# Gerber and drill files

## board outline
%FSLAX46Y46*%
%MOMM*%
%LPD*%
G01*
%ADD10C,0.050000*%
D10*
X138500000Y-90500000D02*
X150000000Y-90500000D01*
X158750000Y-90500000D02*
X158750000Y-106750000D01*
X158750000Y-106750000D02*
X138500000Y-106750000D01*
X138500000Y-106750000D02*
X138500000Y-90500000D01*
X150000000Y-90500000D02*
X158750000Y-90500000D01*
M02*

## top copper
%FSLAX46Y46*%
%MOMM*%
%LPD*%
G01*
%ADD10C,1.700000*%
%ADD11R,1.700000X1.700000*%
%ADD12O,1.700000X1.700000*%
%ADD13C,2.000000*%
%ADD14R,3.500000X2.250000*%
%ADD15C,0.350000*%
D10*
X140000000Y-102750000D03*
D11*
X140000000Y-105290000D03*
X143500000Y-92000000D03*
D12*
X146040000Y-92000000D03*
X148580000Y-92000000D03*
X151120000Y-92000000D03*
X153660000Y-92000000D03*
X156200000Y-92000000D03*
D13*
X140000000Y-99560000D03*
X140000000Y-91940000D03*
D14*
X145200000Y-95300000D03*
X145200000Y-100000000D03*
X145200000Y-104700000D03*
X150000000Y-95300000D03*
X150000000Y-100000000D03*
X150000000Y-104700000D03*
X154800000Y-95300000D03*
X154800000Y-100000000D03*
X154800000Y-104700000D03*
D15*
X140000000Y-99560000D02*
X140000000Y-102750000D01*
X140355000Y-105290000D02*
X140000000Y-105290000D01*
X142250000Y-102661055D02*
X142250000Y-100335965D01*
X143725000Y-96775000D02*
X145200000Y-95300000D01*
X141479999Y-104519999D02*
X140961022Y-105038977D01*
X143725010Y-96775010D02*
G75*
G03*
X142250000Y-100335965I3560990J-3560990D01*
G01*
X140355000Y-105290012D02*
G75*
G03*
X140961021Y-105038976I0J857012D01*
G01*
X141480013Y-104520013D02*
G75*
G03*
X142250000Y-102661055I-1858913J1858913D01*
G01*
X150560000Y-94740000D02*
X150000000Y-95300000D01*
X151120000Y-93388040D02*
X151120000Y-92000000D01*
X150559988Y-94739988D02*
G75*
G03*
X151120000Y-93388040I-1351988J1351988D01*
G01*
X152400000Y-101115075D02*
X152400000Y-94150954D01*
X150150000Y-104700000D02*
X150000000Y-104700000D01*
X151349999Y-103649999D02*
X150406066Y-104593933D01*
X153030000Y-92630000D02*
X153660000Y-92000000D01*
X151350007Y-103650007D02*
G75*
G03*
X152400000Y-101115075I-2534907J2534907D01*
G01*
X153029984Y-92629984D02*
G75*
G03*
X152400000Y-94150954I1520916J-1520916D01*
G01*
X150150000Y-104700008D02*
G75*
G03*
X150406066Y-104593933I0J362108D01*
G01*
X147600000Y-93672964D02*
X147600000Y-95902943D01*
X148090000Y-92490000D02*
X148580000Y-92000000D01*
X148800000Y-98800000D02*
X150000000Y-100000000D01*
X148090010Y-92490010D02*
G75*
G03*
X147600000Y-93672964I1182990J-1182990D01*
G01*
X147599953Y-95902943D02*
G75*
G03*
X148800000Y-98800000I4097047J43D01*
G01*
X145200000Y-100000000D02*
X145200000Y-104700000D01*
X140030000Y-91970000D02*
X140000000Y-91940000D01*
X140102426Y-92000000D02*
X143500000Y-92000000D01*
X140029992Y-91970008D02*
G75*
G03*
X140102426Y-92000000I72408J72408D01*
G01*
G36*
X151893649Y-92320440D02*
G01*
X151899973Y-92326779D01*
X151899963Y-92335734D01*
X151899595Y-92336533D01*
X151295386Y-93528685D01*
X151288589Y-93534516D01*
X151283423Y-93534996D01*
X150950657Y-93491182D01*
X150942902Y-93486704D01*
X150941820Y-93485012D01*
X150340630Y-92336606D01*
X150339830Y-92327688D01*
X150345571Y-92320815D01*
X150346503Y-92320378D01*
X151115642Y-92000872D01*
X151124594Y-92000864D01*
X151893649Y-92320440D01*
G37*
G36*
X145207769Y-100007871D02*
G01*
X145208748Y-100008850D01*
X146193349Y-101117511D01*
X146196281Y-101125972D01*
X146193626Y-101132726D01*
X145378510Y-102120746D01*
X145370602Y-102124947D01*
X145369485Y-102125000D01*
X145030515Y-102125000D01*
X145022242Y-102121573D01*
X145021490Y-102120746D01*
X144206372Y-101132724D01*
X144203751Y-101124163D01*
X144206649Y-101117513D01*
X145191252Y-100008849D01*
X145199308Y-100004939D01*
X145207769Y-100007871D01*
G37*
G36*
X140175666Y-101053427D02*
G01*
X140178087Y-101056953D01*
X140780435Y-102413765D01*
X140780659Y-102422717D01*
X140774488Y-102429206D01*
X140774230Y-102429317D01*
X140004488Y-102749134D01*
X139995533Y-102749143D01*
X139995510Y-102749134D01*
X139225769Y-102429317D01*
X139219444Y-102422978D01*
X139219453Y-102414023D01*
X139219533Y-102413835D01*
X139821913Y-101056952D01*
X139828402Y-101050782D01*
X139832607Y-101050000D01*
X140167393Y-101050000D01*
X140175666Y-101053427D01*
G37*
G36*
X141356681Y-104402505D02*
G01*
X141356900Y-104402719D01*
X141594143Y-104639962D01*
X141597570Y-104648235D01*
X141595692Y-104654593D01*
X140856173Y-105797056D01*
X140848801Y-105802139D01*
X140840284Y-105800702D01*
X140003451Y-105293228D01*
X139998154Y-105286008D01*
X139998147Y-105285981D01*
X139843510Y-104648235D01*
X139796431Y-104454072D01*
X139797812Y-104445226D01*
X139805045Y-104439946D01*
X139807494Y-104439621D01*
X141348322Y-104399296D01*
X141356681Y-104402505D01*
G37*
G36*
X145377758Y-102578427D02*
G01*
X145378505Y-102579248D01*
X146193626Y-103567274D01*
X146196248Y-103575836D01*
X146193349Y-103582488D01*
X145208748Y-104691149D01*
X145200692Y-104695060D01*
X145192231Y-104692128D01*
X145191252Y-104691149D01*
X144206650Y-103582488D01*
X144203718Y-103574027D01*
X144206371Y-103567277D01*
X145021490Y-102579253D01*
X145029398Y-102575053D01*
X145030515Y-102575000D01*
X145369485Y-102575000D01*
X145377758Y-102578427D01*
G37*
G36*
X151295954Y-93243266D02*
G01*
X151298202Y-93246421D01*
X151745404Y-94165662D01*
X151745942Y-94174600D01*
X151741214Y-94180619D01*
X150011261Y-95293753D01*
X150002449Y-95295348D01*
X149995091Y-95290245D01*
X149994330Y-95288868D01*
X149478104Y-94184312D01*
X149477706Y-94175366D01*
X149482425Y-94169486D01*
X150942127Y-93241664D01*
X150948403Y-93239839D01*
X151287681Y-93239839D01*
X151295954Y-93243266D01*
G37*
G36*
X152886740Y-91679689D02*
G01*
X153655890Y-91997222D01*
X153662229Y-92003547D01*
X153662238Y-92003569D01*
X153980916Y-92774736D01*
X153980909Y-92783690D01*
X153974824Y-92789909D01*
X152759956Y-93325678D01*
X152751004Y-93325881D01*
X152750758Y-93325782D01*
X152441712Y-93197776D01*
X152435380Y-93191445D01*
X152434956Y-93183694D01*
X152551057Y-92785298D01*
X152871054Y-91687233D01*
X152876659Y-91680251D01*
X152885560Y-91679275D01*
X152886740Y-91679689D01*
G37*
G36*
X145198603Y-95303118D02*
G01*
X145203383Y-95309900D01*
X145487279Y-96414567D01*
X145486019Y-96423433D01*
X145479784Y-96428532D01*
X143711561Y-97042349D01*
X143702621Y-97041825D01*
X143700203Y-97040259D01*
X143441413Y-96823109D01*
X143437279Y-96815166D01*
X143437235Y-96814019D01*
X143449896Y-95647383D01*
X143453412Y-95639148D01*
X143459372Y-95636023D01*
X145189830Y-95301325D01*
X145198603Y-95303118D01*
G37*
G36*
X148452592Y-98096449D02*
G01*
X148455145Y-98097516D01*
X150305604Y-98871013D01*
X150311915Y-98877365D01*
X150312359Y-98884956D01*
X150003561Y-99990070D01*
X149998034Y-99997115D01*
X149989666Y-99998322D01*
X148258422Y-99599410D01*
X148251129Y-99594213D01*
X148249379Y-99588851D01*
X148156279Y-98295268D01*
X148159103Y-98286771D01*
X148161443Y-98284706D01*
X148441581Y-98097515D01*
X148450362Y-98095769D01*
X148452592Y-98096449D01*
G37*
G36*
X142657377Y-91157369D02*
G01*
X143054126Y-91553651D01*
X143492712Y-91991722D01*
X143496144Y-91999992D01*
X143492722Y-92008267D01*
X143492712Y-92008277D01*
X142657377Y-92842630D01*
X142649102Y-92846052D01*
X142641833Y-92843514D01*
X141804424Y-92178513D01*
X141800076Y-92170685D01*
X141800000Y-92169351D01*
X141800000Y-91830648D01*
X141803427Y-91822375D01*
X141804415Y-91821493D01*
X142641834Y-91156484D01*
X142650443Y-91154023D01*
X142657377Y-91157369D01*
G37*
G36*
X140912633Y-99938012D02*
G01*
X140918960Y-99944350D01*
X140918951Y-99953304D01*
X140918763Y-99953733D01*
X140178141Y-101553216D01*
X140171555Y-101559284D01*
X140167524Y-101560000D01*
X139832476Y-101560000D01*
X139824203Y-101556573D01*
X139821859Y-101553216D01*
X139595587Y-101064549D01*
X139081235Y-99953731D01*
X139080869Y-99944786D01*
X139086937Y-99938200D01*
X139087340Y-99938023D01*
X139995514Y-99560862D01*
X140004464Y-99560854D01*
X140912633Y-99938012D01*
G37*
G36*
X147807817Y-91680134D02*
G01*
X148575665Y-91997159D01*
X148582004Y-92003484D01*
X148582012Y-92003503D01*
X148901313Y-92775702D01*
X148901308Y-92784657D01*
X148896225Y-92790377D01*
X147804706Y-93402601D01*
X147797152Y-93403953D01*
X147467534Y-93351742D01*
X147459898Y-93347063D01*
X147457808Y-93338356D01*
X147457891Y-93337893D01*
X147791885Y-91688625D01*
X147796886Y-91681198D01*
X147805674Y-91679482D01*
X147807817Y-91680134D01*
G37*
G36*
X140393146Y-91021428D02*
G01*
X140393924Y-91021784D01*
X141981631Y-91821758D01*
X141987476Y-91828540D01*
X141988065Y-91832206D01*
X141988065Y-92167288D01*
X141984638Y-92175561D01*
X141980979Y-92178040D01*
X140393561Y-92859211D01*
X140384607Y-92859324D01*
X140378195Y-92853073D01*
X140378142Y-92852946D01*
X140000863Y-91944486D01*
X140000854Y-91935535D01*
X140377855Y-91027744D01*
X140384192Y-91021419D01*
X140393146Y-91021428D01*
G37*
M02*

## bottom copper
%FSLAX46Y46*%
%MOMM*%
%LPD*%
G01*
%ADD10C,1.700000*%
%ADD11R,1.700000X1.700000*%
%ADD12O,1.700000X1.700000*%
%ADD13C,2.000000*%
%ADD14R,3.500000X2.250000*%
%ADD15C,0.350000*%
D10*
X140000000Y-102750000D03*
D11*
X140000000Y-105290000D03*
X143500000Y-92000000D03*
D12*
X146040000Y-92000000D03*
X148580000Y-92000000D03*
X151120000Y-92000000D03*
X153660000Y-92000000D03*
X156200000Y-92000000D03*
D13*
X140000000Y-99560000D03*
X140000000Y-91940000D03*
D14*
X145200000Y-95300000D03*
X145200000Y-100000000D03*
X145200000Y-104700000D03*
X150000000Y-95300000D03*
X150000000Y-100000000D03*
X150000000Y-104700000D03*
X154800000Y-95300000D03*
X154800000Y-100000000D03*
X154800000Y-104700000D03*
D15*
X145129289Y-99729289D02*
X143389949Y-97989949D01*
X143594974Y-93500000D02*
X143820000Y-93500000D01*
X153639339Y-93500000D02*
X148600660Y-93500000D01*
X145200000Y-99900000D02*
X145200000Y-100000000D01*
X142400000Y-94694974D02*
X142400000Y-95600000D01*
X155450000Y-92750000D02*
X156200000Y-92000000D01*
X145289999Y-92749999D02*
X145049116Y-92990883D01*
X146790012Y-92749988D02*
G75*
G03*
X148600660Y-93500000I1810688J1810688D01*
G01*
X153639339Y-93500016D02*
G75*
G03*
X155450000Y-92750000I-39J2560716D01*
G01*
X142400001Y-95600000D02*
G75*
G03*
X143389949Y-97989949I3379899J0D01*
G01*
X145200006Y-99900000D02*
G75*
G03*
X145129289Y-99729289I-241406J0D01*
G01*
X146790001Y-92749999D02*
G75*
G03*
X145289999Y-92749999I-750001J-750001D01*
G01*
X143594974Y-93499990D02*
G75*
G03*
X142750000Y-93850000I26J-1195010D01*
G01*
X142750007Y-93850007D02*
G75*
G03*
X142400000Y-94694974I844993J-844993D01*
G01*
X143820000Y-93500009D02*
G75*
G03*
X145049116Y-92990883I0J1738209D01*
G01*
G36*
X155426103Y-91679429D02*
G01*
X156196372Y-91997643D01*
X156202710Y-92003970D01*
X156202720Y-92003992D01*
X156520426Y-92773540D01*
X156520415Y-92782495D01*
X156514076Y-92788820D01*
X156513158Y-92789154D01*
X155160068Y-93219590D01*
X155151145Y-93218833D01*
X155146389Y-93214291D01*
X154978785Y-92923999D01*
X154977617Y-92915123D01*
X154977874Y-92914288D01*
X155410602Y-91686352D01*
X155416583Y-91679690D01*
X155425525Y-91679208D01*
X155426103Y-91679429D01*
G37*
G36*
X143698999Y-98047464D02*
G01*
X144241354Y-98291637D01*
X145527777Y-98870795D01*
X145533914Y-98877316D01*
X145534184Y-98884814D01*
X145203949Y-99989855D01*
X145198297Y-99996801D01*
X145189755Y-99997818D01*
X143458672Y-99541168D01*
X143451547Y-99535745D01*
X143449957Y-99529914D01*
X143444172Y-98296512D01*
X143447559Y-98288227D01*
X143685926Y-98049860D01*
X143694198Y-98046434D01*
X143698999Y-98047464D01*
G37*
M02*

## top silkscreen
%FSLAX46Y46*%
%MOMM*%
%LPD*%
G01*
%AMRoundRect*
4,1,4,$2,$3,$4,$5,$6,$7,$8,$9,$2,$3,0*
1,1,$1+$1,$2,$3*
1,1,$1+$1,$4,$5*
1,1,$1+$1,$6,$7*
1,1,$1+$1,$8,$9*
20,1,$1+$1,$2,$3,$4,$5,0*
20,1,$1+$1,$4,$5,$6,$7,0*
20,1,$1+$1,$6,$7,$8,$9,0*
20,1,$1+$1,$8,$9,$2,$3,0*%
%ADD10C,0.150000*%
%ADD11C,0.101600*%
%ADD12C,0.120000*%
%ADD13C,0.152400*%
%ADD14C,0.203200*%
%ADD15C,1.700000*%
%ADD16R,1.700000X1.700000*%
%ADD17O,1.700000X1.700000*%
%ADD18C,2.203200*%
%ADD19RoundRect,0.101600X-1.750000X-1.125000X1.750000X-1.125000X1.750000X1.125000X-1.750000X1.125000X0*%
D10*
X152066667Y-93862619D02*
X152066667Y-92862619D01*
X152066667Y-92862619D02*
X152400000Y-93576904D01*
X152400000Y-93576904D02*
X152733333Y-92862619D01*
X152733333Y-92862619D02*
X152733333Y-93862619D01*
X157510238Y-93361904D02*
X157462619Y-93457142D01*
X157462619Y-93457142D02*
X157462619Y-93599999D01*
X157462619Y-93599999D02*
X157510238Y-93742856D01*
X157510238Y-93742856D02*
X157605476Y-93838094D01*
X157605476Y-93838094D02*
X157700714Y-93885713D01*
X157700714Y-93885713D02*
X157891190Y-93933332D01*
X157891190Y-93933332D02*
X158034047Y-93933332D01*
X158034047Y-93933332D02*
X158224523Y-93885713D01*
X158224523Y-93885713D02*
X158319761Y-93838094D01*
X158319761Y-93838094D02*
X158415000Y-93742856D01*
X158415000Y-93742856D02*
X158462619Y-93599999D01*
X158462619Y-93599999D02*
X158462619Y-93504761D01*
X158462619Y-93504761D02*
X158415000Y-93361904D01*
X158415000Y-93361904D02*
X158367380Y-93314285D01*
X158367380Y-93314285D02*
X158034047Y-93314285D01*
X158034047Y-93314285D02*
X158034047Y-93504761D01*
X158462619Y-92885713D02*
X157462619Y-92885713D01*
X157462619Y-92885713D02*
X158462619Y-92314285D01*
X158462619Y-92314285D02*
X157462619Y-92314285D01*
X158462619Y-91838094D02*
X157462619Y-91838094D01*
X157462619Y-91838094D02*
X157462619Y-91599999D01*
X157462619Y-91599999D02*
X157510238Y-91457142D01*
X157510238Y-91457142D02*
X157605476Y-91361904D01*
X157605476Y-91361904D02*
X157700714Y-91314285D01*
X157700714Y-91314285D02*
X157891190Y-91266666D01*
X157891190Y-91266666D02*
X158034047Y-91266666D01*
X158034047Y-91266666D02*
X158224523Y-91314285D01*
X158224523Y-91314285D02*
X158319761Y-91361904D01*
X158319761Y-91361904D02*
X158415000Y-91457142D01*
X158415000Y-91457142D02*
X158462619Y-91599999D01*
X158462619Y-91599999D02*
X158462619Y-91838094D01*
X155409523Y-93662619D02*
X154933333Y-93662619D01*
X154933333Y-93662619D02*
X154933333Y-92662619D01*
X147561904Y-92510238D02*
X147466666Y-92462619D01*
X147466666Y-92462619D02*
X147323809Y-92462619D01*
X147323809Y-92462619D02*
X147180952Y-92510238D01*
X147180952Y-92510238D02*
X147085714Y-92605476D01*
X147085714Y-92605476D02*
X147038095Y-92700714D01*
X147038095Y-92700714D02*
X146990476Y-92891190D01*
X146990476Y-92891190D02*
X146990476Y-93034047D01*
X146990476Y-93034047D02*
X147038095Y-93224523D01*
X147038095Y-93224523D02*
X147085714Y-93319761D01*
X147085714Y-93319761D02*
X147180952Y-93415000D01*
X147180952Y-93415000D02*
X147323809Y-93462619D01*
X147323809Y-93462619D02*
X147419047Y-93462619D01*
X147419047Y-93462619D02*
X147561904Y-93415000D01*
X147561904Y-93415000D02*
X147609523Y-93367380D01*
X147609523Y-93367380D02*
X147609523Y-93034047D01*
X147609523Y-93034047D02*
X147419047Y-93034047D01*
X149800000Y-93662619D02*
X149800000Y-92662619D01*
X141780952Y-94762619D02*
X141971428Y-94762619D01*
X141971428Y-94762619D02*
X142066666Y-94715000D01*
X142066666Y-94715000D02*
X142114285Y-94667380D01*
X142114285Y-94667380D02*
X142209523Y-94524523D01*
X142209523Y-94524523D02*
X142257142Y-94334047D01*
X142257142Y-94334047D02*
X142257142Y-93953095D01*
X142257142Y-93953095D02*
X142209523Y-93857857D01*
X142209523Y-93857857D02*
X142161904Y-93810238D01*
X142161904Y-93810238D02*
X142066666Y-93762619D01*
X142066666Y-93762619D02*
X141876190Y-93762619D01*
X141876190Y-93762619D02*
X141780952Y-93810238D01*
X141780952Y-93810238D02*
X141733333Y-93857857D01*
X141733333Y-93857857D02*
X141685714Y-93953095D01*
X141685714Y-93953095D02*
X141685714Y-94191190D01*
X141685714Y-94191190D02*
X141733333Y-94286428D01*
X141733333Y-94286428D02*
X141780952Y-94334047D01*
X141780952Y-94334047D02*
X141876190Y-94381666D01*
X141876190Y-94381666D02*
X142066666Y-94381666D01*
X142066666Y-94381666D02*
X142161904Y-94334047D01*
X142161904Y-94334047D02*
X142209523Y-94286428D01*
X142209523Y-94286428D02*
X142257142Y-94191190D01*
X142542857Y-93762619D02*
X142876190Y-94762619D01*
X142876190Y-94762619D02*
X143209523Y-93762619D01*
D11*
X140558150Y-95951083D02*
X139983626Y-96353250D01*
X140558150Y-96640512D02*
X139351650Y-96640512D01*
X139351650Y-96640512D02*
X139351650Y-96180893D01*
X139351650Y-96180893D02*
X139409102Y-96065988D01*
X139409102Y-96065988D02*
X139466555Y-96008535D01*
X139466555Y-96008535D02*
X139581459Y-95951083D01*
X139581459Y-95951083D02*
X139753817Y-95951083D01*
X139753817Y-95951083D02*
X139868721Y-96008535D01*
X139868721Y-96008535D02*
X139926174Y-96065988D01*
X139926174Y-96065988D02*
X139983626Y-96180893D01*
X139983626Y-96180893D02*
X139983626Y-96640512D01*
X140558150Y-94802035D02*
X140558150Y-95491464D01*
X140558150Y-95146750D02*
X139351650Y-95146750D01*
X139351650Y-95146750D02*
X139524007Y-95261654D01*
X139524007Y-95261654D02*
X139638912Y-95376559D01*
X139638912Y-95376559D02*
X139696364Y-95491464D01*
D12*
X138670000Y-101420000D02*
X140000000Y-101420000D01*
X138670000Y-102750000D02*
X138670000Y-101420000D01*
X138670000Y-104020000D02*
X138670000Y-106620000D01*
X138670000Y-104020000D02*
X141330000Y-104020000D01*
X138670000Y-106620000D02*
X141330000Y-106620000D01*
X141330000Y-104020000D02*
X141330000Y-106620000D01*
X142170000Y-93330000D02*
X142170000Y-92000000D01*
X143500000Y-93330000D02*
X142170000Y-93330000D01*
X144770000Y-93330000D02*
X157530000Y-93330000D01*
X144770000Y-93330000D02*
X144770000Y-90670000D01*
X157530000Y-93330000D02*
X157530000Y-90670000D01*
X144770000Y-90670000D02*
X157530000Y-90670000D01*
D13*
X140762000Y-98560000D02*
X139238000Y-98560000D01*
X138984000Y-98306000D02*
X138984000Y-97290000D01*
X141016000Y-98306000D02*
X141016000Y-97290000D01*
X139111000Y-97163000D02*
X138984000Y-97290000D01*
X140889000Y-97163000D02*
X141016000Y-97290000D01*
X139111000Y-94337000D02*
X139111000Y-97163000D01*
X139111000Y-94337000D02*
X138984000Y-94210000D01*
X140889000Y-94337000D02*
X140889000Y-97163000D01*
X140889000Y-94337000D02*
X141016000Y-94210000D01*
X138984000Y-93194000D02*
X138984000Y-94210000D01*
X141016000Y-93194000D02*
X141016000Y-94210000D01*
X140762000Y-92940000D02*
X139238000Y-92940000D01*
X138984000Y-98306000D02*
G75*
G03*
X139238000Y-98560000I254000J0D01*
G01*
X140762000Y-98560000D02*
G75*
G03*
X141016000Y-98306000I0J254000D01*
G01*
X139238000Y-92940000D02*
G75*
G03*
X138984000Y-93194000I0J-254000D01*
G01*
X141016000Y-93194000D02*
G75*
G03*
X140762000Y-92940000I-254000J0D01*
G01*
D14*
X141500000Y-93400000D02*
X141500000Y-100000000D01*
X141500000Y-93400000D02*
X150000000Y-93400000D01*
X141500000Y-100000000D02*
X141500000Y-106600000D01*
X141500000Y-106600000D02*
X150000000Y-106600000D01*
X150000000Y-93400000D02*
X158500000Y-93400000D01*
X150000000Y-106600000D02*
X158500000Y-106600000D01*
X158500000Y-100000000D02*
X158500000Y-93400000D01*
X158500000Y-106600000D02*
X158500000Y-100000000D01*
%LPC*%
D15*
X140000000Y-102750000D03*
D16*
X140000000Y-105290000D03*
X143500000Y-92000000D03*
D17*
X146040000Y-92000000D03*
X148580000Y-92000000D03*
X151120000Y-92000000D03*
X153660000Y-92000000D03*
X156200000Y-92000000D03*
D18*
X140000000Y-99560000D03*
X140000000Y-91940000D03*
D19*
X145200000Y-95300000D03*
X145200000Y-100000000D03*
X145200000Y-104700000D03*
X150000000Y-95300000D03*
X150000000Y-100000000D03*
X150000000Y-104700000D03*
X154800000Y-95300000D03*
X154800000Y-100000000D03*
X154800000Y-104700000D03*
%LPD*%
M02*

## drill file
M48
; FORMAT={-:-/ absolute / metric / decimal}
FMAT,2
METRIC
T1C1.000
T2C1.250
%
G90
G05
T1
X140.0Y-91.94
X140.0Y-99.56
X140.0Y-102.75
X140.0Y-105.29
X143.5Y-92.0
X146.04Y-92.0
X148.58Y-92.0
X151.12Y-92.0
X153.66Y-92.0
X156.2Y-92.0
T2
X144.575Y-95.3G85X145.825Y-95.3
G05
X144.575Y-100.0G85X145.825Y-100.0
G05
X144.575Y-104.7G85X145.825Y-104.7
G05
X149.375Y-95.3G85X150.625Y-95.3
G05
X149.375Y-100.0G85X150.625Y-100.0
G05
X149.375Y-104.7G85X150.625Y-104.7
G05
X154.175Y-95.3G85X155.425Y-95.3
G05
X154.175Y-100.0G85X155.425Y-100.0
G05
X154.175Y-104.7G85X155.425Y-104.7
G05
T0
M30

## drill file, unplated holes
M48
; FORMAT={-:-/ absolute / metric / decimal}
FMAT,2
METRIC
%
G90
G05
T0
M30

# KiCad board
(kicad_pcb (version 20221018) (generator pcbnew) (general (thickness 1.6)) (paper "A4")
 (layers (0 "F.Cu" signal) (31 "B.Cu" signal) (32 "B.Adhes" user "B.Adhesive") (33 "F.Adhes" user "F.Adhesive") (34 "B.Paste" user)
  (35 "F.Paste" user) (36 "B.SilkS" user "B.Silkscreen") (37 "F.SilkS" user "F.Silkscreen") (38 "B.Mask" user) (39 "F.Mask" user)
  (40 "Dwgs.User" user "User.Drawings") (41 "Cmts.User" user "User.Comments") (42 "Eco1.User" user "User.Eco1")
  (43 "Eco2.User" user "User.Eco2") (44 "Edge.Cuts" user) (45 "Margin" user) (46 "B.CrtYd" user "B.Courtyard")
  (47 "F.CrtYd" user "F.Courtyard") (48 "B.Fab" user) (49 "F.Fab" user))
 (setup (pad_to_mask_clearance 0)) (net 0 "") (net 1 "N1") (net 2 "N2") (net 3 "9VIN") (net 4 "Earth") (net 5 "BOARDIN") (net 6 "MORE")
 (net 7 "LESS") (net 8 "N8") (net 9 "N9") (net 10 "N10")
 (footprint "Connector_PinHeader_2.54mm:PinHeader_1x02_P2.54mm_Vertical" (layer "F.Cu") (at 140 102.75)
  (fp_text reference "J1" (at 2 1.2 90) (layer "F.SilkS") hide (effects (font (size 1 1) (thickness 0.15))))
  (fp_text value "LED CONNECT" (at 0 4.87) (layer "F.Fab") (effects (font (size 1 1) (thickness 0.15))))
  (fp_line (start -1.33 -1.33) (end 0 -1.33) (stroke (width 0.12) (type solid)) (layer "F.SilkS"))
  (fp_line (start -1.33 0) (end -1.33 -1.33) (stroke (width 0.12) (type solid)) (layer "F.SilkS"))
  (fp_line (start -1.33 1.27) (end -1.33 3.87) (stroke (width 0.12) (type solid)) (layer "F.SilkS"))
  (fp_line (start -1.33 1.27) (end 1.33 1.27) (stroke (width 0.12) (type solid)) (layer "F.SilkS"))
  (fp_line (start -1.33 3.87) (end 1.33 3.87) (stroke (width 0.12) (type solid)) (layer "F.SilkS"))
  (fp_line (start 1.33 1.27) (end 1.33 3.87) (stroke (width 0.12) (type solid)) (layer "F.SilkS"))
  (pad "1" thru_hole circle (at 0 0) (size 1.7 1.7) (drill 1) (layers "*.Cu" "*.Mask") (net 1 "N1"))
  (pad "2" thru_hole rect (at 0 2.54) (size 1.7 1.7) (drill 1) (layers "*.Cu" "*.Mask") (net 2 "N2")))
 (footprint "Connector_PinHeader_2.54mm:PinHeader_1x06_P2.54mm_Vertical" (layer "F.Cu") (at 143.5 92 90)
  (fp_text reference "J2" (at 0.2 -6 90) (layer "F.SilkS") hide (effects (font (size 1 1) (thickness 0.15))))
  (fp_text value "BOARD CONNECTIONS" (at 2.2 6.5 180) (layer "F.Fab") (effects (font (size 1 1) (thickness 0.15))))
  (fp_line (start -1.33 -1.33) (end 0 -1.33) (stroke (width 0.12) (type solid)) (layer "F.SilkS"))
  (fp_line (start -1.33 0) (end -1.33 -1.33) (stroke (width 0.12) (type solid)) (layer "F.SilkS"))
  (fp_line (start -1.33 1.27) (end -1.33 14.03) (stroke (width 0.12) (type solid)) (layer "F.SilkS"))
  (fp_line (start -1.33 1.27) (end 1.33 1.27) (stroke (width 0.12) (type solid)) (layer "F.SilkS"))
  (fp_line (start -1.33 14.03) (end 1.33 14.03) (stroke (width 0.12) (type solid)) (layer "F.SilkS"))
  (fp_line (start 1.33 1.27) (end 1.33 14.03) (stroke (width 0.12) (type solid)) (layer "F.SilkS"))
  (pad "1" thru_hole rect (at 0 0 90) (size 1.7 1.7) (drill 1) (layers "*.Cu" "*.Mask") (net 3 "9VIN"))
  (pad "2" thru_hole oval (at 0 2.54 90) (size 1.7 1.7) (drill 1) (layers "*.Cu" "*.Mask") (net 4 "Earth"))
  (pad "3" thru_hole oval (at 0 5.08 90) (size 1.7 1.7) (drill 1) (layers "*.Cu" "*.Mask") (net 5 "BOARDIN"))
  (pad "4" thru_hole oval (at 0 7.62 90) (size 1.7 1.7) (drill 1) (layers "*.Cu" "*.Mask") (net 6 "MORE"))
  (pad "5" thru_hole oval (at 0 10.16 90) (size 1.7 1.7) (drill 1) (layers "*.Cu" "*.Mask") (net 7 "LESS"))
  (pad "6" thru_hole oval (at 0 12.7 90) (size 1.7 1.7) (drill 1) (layers "*.Cu" "*.Mask") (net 4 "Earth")))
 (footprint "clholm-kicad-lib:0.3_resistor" (layer "F.Cu") (at 140 95.75 90)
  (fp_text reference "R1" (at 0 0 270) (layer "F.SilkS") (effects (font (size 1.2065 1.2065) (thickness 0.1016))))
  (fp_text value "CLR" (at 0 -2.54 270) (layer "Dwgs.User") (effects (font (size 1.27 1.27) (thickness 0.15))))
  (fp_line (start -2.81 0.762) (end -2.81 -0.762) (stroke (width 0.1524) (type solid)) (layer "F.SilkS"))
  (fp_line (start -2.556 -1.016) (end -1.54 -1.016) (stroke (width 0.1524) (type solid)) (layer "F.SilkS"))
  (fp_line (start -2.556 1.016) (end -1.54 1.016) (stroke (width 0.1524) (type solid)) (layer "F.SilkS"))
  (fp_line (start -1.413 -0.889) (end -1.54 -1.016) (stroke (width 0.1524) (type solid)) (layer "F.SilkS"))
  (fp_line (start -1.413 0.889) (end -1.54 1.016) (stroke (width 0.1524) (type solid)) (layer "F.SilkS"))
  (fp_line (start 1.413 -0.889) (end -1.413 -0.889) (stroke (width 0.1524) (type solid)) (layer "F.SilkS"))
  (fp_line (start 1.413 -0.889) (end 1.54 -1.016) (stroke (width 0.1524) (type solid)) (layer "F.SilkS"))
  (fp_line (start 1.413 0.889) (end -1.413 0.889) (stroke (width 0.1524) (type solid)) (layer "F.SilkS"))
  (fp_line (start 1.413 0.889) (end 1.54 1.016) (stroke (width 0.1524) (type solid)) (layer "F.SilkS"))
  (fp_line (start 2.556 -1.016) (end 1.54 -1.016) (stroke (width 0.1524) (type solid)) (layer "F.SilkS"))
  (fp_line (start 2.556 1.016) (end 1.54 1.016) (stroke (width 0.1524) (type solid)) (layer "F.SilkS"))
  (fp_line (start 2.81 0.762) (end 2.81 -0.762) (stroke (width 0.1524) (type solid)) (layer "F.SilkS"))
  (fp_arc (start -2.81 -0.762) (mid -2.735605 -0.941605) (end -2.556 -1.016) (stroke (width 0.1524) (type solid)) (layer "F.SilkS"))
  (fp_arc (start -2.556 1.016) (mid -2.735605 0.941605) (end -2.81 0.762) (stroke (width 0.1524) (type solid)) (layer "F.SilkS"))
  (fp_arc (start 2.556 -1.016) (mid 2.735605 -0.941605) (end 2.81 -0.762) (stroke (width 0.1524) (type solid)) (layer "F.SilkS"))
  (fp_arc (start 2.81 0.762) (mid 2.735605 0.941605) (end 2.556 1.016) (stroke (width 0.1524) (type solid)) (layer "F.SilkS"))
  (pad "1" thru_hole circle (at -3.81 0 90) (size 2 2) (drill 1) (layers "*.Cu" "*.Mask") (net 1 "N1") (solder_mask_margin 0.1016))
  (pad "2" thru_hole circle (at 3.81 0 90) (size 2 2) (drill 1) (layers "*.Cu" "*.Mask") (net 3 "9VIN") (solder_mask_margin 0.1016)))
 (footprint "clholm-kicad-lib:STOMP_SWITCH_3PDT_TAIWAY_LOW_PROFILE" (layer "F.Cu") (at 150 100)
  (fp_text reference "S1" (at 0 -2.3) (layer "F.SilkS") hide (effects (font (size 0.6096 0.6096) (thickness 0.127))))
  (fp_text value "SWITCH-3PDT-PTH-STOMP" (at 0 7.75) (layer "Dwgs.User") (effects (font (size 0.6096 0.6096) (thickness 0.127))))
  (fp_line (start -8.5 -6.6) (end -8.5 0) (stroke (width 0.2032) (type solid)) (layer "F.SilkS"))
  (fp_line (start -8.5 -6.6) (end 0 -6.6) (stroke (width 0.2032) (type solid)) (layer "F.SilkS"))
  (fp_line (start -8.5 0) (end -8.5 6.6) (stroke (width 0.2032) (type solid)) (layer "F.SilkS"))
  (fp_line (start -8.5 6.6) (end 0 6.6) (stroke (width 0.2032) (type solid)) (layer "F.SilkS"))
  (fp_line (start 0 -6.6) (end 8.5 -6.6) (stroke (width 0.2032) (type solid)) (layer "F.SilkS"))
  (fp_line (start 0 6.6) (end 8.5 6.6) (stroke (width 0.2032) (type solid)) (layer "F.SilkS"))
  (fp_line (start 8.5 0) (end 8.5 -6.6) (stroke (width 0.2032) (type solid)) (layer "F.SilkS"))
  (fp_line (start 8.5 6.6) (end 8.5 0) (stroke (width 0.2032) (type solid)) (layer "F.SilkS"))
  (pad "P$1" thru_hole rect (at -4.8 -4.7) (size 3.5 2.25) (drill oval 2.5 1.25) (layers "*.Cu" "*.Mask") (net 2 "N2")
   (solder_mask_margin 0.1016))
  (pad "P$2" thru_hole rect (at -4.8 0) (size 3.5 2.25) (drill oval 2.5 1.25) (layers "*.Cu" "*.Mask") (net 4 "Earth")
   (solder_mask_margin 0.1016))
  (pad "P$3" thru_hole rect (at -4.8 4.7) (size 3.5 2.25) (drill oval 2.5 1.25) (layers "*.Cu" "*.Mask") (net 4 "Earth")
   (solder_mask_margin 0.1016))
  (pad "P$4" thru_hole rect (at 0 -4.7) (size 3.5 2.25) (drill oval 2.5 1.25) (layers "*.Cu" "*.Mask") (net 6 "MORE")
   (solder_mask_margin 0.1016))
  (pad "P$5" thru_hole rect (at 0 0) (size 3.5 2.25) (drill oval 2.5 1.25) (layers "*.Cu" "*.Mask") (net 5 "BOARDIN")
   (solder_mask_margin 0.1016))
  (pad "P$6" thru_hole rect (at 0 4.7) (size 3.5 2.25) (drill oval 2.5 1.25) (layers "*.Cu" "*.Mask") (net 7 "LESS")
   (solder_mask_margin 0.1016))
  (pad "P$7" thru_hole rect (at 4.8 -4.7) (size 3.5 2.25) (drill oval 2.5 1.25) (layers "*.Cu" "*.Mask") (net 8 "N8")
   (solder_mask_margin 0.1016))
  (pad "P$8" thru_hole rect (at 4.8 0) (size 3.5 2.25) (drill oval 2.5 1.25) (layers "*.Cu" "*.Mask") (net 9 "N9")
   (solder_mask_margin 0.1016))
  (pad "P$9" thru_hole rect (at 4.8 4.7) (size 3.5 2.25) (drill oval 2.5 1.25) (layers "*.Cu" "*.Mask") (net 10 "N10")
   (solder_mask_margin 0.1016)))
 (gr_line (start 138.5 90.5) (end 150 90.5) (stroke (width 0.05) (type solid)) (layer "Edge.Cuts"))
 (gr_line (start 158.75 90.5) (end 158.75 106.75) (stroke (width 0.05) (type solid)) (layer "Edge.Cuts"))
 (gr_line (start 158.75 106.75) (end 138.5 106.75) (stroke (width 0.05) (type solid)) (layer "Edge.Cuts"))
 (gr_line (start 138.5 106.75) (end 138.5 90.5) (stroke (width 0.05) (type solid)) (layer "Edge.Cuts"))
 (gr_line (start 150 90.5) (end 158.75 90.5) (stroke (width 0.05) (type solid)) (layer "Edge.Cuts"))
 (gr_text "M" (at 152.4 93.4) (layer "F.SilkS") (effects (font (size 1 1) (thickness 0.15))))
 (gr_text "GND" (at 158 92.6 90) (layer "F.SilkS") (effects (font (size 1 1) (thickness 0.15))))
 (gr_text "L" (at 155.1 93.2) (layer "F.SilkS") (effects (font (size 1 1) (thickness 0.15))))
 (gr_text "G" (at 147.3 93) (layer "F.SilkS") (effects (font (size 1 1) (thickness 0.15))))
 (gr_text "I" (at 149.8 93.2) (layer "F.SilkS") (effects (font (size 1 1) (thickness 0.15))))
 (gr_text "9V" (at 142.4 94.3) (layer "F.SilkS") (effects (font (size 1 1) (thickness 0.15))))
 (segment (start 140 99.56) (end 140 102.75) (width 0.35) (layer "F.Cu") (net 1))
 (segment (start 140.355 105.29) (end 140 105.29) (width 0.35) (layer "F.Cu") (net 2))
 (segment (start 142.25 102.661055) (end 142.25 100.335965) (width 0.35) (layer "F.Cu") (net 2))
 (segment (start 143.725 96.775) (end 145.2 95.3) (width 0.35) (layer "F.Cu") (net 2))
 (segment (start 141.479999 104.519999) (end 140.961022 105.038977) (width 0.35) (layer "F.Cu") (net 2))
 (arc (start 143.725 96.775) (mid 142.63334 98.408784) (end 142.25 100.335965) (width 0.35) (layer "F.Cu") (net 2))
 (arc (start 140.961022 105.038977) (mid 140.682976 105.224761) (end 140.355 105.29) (width 0.35) (layer "F.Cu") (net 2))
 (arc (start 142.25 102.661055) (mid 142.049883 103.667108) (end 141.479999 104.519999) (width 0.35) (layer "F.Cu") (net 2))
 (segment (start 150.56 94.74) (end 150 95.3) (width 0.35) (layer "F.Cu") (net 6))
 (segment (start 151.12 93.38804) (end 151.12 92) (width 0.35) (layer "F.Cu") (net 6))
 (arc (start 151.12 93.38804) (mid 150.97446 94.119715) (end 150.56 94.74) (width 0.35) (layer "F.Cu") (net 6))
 (segment (start 152.4 101.115075) (end 152.4 94.150954) (width 0.35) (layer "F.Cu") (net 7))
 (segment (start 150.15 104.7) (end 150 104.7) (width 0.35) (layer "F.Cu") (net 7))
 (segment (start 151.349999 103.649999) (end 150.406066 104.593933) (width 0.35) (layer "F.Cu") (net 7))
 (segment (start 153.03 92.63) (end 153.66 92) (width 0.35) (layer "F.Cu") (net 7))
 (arc (start 152.4 101.115075) (mid 152.127113 102.486966) (end 151.349999 103.649999) (width 0.35) (layer "F.Cu") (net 7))
 (arc (start 153.03 92.63) (mid 152.563731 93.327819) (end 152.4 94.150954) (width 0.35) (layer "F.Cu") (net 7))
 (arc (start 150.406066 104.593933) (mid 150.288581 104.672434) (end 150.15 104.7) (width 0.35) (layer "F.Cu") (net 7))
 (segment (start 147.6 93.672964) (end 147.6 95.902943) (width 0.35) (layer "F.Cu") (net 5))
 (segment (start 148.09 92.49) (end 148.58 92) (width 0.35) (layer "F.Cu") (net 5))
 (segment (start 148.8 98.8) (end 150 100) (width 0.35) (layer "F.Cu") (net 5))
 (arc (start 148.09 92.49) (mid 147.727346 93.032748) (end 147.6 93.672964) (width 0.35) (layer "F.Cu") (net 5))
 (arc (start 147.6 95.902943) (mid 147.911869 97.470819) (end 148.8 98.8) (width 0.35) (layer "F.Cu") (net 5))
 (segment (start 145.2 100) (end 145.2 104.7) (width 0.35) (layer "F.Cu") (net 4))
 (segment (start 145.129289 99.729289) (end 143.389949 97.989949) (width 0.35) (layer "B.Cu") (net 4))
 (segment (start 143.594974 93.5) (end 143.82 93.5) (width 0.35) (layer "B.Cu") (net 4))
 (segment (start 153.639339 93.5) (end 148.60066 93.5) (width 0.35) (layer "B.Cu") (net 4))
 (segment (start 145.2 99.9) (end 145.2 100) (width 0.35) (layer "B.Cu") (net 4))
 (segment (start 142.4 94.694974) (end 142.4 95.6) (width 0.35) (layer "B.Cu") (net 4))
 (segment (start 155.45 92.75) (end 156.2 92) (width 0.35) (layer "B.Cu") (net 4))
 (segment (start 145.289999 92.749999) (end 145.049116 92.990883) (width 0.35) (layer "B.Cu") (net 4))
 (arc (start 146.79 92.75) (mid 147.620737 93.305081) (end 148.60066 93.5) (width 0.35) (layer "B.Cu") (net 4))
 (arc (start 155.45 92.75) (mid 154.619261 93.305081) (end 153.639339 93.5) (width 0.35) (layer "B.Cu") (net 4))
 (arc (start 142.4 95.6) (mid 142.657279 96.893431) (end 143.389949 97.989949) (width 0.35) (layer "B.Cu") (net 4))
 (arc (start 145.129289 99.729289) (mid 145.181622 99.807611) (end 145.2 99.9) (width 0.35) (layer "B.Cu") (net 4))
 (arc (start 146.79 92.75) (mid 146.039999 92.439339) (end 145.289999 92.749999) (width 0.35) (layer "B.Cu") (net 4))
 (arc (start 143.594974 93.5) (mid 143.137677 93.590962) (end 142.75 93.85) (width 0.35) (layer "B.Cu") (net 4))
 (arc (start 142.75 93.85) (mid 142.490962 94.237677) (end 142.4 94.694974) (width 0.35) (layer "B.Cu") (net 4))
 (arc (start 145.049116 92.990883) (mid 144.485193 93.367684) (end 143.82 93.5) (width 0.35) (layer "B.Cu") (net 4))
 (segment (start 140.03 91.97) (end 140 91.94) (width 0.35) (layer "F.Cu") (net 3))
 (segment (start 140.102426 92) (end 143.5 92) (width 0.35) (layer "F.Cu") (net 3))
 (arc (start 140.03 91.97) (mid 140.063229 91.992203) (end 140.102426 92) (width 0.35) (layer "F.Cu") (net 3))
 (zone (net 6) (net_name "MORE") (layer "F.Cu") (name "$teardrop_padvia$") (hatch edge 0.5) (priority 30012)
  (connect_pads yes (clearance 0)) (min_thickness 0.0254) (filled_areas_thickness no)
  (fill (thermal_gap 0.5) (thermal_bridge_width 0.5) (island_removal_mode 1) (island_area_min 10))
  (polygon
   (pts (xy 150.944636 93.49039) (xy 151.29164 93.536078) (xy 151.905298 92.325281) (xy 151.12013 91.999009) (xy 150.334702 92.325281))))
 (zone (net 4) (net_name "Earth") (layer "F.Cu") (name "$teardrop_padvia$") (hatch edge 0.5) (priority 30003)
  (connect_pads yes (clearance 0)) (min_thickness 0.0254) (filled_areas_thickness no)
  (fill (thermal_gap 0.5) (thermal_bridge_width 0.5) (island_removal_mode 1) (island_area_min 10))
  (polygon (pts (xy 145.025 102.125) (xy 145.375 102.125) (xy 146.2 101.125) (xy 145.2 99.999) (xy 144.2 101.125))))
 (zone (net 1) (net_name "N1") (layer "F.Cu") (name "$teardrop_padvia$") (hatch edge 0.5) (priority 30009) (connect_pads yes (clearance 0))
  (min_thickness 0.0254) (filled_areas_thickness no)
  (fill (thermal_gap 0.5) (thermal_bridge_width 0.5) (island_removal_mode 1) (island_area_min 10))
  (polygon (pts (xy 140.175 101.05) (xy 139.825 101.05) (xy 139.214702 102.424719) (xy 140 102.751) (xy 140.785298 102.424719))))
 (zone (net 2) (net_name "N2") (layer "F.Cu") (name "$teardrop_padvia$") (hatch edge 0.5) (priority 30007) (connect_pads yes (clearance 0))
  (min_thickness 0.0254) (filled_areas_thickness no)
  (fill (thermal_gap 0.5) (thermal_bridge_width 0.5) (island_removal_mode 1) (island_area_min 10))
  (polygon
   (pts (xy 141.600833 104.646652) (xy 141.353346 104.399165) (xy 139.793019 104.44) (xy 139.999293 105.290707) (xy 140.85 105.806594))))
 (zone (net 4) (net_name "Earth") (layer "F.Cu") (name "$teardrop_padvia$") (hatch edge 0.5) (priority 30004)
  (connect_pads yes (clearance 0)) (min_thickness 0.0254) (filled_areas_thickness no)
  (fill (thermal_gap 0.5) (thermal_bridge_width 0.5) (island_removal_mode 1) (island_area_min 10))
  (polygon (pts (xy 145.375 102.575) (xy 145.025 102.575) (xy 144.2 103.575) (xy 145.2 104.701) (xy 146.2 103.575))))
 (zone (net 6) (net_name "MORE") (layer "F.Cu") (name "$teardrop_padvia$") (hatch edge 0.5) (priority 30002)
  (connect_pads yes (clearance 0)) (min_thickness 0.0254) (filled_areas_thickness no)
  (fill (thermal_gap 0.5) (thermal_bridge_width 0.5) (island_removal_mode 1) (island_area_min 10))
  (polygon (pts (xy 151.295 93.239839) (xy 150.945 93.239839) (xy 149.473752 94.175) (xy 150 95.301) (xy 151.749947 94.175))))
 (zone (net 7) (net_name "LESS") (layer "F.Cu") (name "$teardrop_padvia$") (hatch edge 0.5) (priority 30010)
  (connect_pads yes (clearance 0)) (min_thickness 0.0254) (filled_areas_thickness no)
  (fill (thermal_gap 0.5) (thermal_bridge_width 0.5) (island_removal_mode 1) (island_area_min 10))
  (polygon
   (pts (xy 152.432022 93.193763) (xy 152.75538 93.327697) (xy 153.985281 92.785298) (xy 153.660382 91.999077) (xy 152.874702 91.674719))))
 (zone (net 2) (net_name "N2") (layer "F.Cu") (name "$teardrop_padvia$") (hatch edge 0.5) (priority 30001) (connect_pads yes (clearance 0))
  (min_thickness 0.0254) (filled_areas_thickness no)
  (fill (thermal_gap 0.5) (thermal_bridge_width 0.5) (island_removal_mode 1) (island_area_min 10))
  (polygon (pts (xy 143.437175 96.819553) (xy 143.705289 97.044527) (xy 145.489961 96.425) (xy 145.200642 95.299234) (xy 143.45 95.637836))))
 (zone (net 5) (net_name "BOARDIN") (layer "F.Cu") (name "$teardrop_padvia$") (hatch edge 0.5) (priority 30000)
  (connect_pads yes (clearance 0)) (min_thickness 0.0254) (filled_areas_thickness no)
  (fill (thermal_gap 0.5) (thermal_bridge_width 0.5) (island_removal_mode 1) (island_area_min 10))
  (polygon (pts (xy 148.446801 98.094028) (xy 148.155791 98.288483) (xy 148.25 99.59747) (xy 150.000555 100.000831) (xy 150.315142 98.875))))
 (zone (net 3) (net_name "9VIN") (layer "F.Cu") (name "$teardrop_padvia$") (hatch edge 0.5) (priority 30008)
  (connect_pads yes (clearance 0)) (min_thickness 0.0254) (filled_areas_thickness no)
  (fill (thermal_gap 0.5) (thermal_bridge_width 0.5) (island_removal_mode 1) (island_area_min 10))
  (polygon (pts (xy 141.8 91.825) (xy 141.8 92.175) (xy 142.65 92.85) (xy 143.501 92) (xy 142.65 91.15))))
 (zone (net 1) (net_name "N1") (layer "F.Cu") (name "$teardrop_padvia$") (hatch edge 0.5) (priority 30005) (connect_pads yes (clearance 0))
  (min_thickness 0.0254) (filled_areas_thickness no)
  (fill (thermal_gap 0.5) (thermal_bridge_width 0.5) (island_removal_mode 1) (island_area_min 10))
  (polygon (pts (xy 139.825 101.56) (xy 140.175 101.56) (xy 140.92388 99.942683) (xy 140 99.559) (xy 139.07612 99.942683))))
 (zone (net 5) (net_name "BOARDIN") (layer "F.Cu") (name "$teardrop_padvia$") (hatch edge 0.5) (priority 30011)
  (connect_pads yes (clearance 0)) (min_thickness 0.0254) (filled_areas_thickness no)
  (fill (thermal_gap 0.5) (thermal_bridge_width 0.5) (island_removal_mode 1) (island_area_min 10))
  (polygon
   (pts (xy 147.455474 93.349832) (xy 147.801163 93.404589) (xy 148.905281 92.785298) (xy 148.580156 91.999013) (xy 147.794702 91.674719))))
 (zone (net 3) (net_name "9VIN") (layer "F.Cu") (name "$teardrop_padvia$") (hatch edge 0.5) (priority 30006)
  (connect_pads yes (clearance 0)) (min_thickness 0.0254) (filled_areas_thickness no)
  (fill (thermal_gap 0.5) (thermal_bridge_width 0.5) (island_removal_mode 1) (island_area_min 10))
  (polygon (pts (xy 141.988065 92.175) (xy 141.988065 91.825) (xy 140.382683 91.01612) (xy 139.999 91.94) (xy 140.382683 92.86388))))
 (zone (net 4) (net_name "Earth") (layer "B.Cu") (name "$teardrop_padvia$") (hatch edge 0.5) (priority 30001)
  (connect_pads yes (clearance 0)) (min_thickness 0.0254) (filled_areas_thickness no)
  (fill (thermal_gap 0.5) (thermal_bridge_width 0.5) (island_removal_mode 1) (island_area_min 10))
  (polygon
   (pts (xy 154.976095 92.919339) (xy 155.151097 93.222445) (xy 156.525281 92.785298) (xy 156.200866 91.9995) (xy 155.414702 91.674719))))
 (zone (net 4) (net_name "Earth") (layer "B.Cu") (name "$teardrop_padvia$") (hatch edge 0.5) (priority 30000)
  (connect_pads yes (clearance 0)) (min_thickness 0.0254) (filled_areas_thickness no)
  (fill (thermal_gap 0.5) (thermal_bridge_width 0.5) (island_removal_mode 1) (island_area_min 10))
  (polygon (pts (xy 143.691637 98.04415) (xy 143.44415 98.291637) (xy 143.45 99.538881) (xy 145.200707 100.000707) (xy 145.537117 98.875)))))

